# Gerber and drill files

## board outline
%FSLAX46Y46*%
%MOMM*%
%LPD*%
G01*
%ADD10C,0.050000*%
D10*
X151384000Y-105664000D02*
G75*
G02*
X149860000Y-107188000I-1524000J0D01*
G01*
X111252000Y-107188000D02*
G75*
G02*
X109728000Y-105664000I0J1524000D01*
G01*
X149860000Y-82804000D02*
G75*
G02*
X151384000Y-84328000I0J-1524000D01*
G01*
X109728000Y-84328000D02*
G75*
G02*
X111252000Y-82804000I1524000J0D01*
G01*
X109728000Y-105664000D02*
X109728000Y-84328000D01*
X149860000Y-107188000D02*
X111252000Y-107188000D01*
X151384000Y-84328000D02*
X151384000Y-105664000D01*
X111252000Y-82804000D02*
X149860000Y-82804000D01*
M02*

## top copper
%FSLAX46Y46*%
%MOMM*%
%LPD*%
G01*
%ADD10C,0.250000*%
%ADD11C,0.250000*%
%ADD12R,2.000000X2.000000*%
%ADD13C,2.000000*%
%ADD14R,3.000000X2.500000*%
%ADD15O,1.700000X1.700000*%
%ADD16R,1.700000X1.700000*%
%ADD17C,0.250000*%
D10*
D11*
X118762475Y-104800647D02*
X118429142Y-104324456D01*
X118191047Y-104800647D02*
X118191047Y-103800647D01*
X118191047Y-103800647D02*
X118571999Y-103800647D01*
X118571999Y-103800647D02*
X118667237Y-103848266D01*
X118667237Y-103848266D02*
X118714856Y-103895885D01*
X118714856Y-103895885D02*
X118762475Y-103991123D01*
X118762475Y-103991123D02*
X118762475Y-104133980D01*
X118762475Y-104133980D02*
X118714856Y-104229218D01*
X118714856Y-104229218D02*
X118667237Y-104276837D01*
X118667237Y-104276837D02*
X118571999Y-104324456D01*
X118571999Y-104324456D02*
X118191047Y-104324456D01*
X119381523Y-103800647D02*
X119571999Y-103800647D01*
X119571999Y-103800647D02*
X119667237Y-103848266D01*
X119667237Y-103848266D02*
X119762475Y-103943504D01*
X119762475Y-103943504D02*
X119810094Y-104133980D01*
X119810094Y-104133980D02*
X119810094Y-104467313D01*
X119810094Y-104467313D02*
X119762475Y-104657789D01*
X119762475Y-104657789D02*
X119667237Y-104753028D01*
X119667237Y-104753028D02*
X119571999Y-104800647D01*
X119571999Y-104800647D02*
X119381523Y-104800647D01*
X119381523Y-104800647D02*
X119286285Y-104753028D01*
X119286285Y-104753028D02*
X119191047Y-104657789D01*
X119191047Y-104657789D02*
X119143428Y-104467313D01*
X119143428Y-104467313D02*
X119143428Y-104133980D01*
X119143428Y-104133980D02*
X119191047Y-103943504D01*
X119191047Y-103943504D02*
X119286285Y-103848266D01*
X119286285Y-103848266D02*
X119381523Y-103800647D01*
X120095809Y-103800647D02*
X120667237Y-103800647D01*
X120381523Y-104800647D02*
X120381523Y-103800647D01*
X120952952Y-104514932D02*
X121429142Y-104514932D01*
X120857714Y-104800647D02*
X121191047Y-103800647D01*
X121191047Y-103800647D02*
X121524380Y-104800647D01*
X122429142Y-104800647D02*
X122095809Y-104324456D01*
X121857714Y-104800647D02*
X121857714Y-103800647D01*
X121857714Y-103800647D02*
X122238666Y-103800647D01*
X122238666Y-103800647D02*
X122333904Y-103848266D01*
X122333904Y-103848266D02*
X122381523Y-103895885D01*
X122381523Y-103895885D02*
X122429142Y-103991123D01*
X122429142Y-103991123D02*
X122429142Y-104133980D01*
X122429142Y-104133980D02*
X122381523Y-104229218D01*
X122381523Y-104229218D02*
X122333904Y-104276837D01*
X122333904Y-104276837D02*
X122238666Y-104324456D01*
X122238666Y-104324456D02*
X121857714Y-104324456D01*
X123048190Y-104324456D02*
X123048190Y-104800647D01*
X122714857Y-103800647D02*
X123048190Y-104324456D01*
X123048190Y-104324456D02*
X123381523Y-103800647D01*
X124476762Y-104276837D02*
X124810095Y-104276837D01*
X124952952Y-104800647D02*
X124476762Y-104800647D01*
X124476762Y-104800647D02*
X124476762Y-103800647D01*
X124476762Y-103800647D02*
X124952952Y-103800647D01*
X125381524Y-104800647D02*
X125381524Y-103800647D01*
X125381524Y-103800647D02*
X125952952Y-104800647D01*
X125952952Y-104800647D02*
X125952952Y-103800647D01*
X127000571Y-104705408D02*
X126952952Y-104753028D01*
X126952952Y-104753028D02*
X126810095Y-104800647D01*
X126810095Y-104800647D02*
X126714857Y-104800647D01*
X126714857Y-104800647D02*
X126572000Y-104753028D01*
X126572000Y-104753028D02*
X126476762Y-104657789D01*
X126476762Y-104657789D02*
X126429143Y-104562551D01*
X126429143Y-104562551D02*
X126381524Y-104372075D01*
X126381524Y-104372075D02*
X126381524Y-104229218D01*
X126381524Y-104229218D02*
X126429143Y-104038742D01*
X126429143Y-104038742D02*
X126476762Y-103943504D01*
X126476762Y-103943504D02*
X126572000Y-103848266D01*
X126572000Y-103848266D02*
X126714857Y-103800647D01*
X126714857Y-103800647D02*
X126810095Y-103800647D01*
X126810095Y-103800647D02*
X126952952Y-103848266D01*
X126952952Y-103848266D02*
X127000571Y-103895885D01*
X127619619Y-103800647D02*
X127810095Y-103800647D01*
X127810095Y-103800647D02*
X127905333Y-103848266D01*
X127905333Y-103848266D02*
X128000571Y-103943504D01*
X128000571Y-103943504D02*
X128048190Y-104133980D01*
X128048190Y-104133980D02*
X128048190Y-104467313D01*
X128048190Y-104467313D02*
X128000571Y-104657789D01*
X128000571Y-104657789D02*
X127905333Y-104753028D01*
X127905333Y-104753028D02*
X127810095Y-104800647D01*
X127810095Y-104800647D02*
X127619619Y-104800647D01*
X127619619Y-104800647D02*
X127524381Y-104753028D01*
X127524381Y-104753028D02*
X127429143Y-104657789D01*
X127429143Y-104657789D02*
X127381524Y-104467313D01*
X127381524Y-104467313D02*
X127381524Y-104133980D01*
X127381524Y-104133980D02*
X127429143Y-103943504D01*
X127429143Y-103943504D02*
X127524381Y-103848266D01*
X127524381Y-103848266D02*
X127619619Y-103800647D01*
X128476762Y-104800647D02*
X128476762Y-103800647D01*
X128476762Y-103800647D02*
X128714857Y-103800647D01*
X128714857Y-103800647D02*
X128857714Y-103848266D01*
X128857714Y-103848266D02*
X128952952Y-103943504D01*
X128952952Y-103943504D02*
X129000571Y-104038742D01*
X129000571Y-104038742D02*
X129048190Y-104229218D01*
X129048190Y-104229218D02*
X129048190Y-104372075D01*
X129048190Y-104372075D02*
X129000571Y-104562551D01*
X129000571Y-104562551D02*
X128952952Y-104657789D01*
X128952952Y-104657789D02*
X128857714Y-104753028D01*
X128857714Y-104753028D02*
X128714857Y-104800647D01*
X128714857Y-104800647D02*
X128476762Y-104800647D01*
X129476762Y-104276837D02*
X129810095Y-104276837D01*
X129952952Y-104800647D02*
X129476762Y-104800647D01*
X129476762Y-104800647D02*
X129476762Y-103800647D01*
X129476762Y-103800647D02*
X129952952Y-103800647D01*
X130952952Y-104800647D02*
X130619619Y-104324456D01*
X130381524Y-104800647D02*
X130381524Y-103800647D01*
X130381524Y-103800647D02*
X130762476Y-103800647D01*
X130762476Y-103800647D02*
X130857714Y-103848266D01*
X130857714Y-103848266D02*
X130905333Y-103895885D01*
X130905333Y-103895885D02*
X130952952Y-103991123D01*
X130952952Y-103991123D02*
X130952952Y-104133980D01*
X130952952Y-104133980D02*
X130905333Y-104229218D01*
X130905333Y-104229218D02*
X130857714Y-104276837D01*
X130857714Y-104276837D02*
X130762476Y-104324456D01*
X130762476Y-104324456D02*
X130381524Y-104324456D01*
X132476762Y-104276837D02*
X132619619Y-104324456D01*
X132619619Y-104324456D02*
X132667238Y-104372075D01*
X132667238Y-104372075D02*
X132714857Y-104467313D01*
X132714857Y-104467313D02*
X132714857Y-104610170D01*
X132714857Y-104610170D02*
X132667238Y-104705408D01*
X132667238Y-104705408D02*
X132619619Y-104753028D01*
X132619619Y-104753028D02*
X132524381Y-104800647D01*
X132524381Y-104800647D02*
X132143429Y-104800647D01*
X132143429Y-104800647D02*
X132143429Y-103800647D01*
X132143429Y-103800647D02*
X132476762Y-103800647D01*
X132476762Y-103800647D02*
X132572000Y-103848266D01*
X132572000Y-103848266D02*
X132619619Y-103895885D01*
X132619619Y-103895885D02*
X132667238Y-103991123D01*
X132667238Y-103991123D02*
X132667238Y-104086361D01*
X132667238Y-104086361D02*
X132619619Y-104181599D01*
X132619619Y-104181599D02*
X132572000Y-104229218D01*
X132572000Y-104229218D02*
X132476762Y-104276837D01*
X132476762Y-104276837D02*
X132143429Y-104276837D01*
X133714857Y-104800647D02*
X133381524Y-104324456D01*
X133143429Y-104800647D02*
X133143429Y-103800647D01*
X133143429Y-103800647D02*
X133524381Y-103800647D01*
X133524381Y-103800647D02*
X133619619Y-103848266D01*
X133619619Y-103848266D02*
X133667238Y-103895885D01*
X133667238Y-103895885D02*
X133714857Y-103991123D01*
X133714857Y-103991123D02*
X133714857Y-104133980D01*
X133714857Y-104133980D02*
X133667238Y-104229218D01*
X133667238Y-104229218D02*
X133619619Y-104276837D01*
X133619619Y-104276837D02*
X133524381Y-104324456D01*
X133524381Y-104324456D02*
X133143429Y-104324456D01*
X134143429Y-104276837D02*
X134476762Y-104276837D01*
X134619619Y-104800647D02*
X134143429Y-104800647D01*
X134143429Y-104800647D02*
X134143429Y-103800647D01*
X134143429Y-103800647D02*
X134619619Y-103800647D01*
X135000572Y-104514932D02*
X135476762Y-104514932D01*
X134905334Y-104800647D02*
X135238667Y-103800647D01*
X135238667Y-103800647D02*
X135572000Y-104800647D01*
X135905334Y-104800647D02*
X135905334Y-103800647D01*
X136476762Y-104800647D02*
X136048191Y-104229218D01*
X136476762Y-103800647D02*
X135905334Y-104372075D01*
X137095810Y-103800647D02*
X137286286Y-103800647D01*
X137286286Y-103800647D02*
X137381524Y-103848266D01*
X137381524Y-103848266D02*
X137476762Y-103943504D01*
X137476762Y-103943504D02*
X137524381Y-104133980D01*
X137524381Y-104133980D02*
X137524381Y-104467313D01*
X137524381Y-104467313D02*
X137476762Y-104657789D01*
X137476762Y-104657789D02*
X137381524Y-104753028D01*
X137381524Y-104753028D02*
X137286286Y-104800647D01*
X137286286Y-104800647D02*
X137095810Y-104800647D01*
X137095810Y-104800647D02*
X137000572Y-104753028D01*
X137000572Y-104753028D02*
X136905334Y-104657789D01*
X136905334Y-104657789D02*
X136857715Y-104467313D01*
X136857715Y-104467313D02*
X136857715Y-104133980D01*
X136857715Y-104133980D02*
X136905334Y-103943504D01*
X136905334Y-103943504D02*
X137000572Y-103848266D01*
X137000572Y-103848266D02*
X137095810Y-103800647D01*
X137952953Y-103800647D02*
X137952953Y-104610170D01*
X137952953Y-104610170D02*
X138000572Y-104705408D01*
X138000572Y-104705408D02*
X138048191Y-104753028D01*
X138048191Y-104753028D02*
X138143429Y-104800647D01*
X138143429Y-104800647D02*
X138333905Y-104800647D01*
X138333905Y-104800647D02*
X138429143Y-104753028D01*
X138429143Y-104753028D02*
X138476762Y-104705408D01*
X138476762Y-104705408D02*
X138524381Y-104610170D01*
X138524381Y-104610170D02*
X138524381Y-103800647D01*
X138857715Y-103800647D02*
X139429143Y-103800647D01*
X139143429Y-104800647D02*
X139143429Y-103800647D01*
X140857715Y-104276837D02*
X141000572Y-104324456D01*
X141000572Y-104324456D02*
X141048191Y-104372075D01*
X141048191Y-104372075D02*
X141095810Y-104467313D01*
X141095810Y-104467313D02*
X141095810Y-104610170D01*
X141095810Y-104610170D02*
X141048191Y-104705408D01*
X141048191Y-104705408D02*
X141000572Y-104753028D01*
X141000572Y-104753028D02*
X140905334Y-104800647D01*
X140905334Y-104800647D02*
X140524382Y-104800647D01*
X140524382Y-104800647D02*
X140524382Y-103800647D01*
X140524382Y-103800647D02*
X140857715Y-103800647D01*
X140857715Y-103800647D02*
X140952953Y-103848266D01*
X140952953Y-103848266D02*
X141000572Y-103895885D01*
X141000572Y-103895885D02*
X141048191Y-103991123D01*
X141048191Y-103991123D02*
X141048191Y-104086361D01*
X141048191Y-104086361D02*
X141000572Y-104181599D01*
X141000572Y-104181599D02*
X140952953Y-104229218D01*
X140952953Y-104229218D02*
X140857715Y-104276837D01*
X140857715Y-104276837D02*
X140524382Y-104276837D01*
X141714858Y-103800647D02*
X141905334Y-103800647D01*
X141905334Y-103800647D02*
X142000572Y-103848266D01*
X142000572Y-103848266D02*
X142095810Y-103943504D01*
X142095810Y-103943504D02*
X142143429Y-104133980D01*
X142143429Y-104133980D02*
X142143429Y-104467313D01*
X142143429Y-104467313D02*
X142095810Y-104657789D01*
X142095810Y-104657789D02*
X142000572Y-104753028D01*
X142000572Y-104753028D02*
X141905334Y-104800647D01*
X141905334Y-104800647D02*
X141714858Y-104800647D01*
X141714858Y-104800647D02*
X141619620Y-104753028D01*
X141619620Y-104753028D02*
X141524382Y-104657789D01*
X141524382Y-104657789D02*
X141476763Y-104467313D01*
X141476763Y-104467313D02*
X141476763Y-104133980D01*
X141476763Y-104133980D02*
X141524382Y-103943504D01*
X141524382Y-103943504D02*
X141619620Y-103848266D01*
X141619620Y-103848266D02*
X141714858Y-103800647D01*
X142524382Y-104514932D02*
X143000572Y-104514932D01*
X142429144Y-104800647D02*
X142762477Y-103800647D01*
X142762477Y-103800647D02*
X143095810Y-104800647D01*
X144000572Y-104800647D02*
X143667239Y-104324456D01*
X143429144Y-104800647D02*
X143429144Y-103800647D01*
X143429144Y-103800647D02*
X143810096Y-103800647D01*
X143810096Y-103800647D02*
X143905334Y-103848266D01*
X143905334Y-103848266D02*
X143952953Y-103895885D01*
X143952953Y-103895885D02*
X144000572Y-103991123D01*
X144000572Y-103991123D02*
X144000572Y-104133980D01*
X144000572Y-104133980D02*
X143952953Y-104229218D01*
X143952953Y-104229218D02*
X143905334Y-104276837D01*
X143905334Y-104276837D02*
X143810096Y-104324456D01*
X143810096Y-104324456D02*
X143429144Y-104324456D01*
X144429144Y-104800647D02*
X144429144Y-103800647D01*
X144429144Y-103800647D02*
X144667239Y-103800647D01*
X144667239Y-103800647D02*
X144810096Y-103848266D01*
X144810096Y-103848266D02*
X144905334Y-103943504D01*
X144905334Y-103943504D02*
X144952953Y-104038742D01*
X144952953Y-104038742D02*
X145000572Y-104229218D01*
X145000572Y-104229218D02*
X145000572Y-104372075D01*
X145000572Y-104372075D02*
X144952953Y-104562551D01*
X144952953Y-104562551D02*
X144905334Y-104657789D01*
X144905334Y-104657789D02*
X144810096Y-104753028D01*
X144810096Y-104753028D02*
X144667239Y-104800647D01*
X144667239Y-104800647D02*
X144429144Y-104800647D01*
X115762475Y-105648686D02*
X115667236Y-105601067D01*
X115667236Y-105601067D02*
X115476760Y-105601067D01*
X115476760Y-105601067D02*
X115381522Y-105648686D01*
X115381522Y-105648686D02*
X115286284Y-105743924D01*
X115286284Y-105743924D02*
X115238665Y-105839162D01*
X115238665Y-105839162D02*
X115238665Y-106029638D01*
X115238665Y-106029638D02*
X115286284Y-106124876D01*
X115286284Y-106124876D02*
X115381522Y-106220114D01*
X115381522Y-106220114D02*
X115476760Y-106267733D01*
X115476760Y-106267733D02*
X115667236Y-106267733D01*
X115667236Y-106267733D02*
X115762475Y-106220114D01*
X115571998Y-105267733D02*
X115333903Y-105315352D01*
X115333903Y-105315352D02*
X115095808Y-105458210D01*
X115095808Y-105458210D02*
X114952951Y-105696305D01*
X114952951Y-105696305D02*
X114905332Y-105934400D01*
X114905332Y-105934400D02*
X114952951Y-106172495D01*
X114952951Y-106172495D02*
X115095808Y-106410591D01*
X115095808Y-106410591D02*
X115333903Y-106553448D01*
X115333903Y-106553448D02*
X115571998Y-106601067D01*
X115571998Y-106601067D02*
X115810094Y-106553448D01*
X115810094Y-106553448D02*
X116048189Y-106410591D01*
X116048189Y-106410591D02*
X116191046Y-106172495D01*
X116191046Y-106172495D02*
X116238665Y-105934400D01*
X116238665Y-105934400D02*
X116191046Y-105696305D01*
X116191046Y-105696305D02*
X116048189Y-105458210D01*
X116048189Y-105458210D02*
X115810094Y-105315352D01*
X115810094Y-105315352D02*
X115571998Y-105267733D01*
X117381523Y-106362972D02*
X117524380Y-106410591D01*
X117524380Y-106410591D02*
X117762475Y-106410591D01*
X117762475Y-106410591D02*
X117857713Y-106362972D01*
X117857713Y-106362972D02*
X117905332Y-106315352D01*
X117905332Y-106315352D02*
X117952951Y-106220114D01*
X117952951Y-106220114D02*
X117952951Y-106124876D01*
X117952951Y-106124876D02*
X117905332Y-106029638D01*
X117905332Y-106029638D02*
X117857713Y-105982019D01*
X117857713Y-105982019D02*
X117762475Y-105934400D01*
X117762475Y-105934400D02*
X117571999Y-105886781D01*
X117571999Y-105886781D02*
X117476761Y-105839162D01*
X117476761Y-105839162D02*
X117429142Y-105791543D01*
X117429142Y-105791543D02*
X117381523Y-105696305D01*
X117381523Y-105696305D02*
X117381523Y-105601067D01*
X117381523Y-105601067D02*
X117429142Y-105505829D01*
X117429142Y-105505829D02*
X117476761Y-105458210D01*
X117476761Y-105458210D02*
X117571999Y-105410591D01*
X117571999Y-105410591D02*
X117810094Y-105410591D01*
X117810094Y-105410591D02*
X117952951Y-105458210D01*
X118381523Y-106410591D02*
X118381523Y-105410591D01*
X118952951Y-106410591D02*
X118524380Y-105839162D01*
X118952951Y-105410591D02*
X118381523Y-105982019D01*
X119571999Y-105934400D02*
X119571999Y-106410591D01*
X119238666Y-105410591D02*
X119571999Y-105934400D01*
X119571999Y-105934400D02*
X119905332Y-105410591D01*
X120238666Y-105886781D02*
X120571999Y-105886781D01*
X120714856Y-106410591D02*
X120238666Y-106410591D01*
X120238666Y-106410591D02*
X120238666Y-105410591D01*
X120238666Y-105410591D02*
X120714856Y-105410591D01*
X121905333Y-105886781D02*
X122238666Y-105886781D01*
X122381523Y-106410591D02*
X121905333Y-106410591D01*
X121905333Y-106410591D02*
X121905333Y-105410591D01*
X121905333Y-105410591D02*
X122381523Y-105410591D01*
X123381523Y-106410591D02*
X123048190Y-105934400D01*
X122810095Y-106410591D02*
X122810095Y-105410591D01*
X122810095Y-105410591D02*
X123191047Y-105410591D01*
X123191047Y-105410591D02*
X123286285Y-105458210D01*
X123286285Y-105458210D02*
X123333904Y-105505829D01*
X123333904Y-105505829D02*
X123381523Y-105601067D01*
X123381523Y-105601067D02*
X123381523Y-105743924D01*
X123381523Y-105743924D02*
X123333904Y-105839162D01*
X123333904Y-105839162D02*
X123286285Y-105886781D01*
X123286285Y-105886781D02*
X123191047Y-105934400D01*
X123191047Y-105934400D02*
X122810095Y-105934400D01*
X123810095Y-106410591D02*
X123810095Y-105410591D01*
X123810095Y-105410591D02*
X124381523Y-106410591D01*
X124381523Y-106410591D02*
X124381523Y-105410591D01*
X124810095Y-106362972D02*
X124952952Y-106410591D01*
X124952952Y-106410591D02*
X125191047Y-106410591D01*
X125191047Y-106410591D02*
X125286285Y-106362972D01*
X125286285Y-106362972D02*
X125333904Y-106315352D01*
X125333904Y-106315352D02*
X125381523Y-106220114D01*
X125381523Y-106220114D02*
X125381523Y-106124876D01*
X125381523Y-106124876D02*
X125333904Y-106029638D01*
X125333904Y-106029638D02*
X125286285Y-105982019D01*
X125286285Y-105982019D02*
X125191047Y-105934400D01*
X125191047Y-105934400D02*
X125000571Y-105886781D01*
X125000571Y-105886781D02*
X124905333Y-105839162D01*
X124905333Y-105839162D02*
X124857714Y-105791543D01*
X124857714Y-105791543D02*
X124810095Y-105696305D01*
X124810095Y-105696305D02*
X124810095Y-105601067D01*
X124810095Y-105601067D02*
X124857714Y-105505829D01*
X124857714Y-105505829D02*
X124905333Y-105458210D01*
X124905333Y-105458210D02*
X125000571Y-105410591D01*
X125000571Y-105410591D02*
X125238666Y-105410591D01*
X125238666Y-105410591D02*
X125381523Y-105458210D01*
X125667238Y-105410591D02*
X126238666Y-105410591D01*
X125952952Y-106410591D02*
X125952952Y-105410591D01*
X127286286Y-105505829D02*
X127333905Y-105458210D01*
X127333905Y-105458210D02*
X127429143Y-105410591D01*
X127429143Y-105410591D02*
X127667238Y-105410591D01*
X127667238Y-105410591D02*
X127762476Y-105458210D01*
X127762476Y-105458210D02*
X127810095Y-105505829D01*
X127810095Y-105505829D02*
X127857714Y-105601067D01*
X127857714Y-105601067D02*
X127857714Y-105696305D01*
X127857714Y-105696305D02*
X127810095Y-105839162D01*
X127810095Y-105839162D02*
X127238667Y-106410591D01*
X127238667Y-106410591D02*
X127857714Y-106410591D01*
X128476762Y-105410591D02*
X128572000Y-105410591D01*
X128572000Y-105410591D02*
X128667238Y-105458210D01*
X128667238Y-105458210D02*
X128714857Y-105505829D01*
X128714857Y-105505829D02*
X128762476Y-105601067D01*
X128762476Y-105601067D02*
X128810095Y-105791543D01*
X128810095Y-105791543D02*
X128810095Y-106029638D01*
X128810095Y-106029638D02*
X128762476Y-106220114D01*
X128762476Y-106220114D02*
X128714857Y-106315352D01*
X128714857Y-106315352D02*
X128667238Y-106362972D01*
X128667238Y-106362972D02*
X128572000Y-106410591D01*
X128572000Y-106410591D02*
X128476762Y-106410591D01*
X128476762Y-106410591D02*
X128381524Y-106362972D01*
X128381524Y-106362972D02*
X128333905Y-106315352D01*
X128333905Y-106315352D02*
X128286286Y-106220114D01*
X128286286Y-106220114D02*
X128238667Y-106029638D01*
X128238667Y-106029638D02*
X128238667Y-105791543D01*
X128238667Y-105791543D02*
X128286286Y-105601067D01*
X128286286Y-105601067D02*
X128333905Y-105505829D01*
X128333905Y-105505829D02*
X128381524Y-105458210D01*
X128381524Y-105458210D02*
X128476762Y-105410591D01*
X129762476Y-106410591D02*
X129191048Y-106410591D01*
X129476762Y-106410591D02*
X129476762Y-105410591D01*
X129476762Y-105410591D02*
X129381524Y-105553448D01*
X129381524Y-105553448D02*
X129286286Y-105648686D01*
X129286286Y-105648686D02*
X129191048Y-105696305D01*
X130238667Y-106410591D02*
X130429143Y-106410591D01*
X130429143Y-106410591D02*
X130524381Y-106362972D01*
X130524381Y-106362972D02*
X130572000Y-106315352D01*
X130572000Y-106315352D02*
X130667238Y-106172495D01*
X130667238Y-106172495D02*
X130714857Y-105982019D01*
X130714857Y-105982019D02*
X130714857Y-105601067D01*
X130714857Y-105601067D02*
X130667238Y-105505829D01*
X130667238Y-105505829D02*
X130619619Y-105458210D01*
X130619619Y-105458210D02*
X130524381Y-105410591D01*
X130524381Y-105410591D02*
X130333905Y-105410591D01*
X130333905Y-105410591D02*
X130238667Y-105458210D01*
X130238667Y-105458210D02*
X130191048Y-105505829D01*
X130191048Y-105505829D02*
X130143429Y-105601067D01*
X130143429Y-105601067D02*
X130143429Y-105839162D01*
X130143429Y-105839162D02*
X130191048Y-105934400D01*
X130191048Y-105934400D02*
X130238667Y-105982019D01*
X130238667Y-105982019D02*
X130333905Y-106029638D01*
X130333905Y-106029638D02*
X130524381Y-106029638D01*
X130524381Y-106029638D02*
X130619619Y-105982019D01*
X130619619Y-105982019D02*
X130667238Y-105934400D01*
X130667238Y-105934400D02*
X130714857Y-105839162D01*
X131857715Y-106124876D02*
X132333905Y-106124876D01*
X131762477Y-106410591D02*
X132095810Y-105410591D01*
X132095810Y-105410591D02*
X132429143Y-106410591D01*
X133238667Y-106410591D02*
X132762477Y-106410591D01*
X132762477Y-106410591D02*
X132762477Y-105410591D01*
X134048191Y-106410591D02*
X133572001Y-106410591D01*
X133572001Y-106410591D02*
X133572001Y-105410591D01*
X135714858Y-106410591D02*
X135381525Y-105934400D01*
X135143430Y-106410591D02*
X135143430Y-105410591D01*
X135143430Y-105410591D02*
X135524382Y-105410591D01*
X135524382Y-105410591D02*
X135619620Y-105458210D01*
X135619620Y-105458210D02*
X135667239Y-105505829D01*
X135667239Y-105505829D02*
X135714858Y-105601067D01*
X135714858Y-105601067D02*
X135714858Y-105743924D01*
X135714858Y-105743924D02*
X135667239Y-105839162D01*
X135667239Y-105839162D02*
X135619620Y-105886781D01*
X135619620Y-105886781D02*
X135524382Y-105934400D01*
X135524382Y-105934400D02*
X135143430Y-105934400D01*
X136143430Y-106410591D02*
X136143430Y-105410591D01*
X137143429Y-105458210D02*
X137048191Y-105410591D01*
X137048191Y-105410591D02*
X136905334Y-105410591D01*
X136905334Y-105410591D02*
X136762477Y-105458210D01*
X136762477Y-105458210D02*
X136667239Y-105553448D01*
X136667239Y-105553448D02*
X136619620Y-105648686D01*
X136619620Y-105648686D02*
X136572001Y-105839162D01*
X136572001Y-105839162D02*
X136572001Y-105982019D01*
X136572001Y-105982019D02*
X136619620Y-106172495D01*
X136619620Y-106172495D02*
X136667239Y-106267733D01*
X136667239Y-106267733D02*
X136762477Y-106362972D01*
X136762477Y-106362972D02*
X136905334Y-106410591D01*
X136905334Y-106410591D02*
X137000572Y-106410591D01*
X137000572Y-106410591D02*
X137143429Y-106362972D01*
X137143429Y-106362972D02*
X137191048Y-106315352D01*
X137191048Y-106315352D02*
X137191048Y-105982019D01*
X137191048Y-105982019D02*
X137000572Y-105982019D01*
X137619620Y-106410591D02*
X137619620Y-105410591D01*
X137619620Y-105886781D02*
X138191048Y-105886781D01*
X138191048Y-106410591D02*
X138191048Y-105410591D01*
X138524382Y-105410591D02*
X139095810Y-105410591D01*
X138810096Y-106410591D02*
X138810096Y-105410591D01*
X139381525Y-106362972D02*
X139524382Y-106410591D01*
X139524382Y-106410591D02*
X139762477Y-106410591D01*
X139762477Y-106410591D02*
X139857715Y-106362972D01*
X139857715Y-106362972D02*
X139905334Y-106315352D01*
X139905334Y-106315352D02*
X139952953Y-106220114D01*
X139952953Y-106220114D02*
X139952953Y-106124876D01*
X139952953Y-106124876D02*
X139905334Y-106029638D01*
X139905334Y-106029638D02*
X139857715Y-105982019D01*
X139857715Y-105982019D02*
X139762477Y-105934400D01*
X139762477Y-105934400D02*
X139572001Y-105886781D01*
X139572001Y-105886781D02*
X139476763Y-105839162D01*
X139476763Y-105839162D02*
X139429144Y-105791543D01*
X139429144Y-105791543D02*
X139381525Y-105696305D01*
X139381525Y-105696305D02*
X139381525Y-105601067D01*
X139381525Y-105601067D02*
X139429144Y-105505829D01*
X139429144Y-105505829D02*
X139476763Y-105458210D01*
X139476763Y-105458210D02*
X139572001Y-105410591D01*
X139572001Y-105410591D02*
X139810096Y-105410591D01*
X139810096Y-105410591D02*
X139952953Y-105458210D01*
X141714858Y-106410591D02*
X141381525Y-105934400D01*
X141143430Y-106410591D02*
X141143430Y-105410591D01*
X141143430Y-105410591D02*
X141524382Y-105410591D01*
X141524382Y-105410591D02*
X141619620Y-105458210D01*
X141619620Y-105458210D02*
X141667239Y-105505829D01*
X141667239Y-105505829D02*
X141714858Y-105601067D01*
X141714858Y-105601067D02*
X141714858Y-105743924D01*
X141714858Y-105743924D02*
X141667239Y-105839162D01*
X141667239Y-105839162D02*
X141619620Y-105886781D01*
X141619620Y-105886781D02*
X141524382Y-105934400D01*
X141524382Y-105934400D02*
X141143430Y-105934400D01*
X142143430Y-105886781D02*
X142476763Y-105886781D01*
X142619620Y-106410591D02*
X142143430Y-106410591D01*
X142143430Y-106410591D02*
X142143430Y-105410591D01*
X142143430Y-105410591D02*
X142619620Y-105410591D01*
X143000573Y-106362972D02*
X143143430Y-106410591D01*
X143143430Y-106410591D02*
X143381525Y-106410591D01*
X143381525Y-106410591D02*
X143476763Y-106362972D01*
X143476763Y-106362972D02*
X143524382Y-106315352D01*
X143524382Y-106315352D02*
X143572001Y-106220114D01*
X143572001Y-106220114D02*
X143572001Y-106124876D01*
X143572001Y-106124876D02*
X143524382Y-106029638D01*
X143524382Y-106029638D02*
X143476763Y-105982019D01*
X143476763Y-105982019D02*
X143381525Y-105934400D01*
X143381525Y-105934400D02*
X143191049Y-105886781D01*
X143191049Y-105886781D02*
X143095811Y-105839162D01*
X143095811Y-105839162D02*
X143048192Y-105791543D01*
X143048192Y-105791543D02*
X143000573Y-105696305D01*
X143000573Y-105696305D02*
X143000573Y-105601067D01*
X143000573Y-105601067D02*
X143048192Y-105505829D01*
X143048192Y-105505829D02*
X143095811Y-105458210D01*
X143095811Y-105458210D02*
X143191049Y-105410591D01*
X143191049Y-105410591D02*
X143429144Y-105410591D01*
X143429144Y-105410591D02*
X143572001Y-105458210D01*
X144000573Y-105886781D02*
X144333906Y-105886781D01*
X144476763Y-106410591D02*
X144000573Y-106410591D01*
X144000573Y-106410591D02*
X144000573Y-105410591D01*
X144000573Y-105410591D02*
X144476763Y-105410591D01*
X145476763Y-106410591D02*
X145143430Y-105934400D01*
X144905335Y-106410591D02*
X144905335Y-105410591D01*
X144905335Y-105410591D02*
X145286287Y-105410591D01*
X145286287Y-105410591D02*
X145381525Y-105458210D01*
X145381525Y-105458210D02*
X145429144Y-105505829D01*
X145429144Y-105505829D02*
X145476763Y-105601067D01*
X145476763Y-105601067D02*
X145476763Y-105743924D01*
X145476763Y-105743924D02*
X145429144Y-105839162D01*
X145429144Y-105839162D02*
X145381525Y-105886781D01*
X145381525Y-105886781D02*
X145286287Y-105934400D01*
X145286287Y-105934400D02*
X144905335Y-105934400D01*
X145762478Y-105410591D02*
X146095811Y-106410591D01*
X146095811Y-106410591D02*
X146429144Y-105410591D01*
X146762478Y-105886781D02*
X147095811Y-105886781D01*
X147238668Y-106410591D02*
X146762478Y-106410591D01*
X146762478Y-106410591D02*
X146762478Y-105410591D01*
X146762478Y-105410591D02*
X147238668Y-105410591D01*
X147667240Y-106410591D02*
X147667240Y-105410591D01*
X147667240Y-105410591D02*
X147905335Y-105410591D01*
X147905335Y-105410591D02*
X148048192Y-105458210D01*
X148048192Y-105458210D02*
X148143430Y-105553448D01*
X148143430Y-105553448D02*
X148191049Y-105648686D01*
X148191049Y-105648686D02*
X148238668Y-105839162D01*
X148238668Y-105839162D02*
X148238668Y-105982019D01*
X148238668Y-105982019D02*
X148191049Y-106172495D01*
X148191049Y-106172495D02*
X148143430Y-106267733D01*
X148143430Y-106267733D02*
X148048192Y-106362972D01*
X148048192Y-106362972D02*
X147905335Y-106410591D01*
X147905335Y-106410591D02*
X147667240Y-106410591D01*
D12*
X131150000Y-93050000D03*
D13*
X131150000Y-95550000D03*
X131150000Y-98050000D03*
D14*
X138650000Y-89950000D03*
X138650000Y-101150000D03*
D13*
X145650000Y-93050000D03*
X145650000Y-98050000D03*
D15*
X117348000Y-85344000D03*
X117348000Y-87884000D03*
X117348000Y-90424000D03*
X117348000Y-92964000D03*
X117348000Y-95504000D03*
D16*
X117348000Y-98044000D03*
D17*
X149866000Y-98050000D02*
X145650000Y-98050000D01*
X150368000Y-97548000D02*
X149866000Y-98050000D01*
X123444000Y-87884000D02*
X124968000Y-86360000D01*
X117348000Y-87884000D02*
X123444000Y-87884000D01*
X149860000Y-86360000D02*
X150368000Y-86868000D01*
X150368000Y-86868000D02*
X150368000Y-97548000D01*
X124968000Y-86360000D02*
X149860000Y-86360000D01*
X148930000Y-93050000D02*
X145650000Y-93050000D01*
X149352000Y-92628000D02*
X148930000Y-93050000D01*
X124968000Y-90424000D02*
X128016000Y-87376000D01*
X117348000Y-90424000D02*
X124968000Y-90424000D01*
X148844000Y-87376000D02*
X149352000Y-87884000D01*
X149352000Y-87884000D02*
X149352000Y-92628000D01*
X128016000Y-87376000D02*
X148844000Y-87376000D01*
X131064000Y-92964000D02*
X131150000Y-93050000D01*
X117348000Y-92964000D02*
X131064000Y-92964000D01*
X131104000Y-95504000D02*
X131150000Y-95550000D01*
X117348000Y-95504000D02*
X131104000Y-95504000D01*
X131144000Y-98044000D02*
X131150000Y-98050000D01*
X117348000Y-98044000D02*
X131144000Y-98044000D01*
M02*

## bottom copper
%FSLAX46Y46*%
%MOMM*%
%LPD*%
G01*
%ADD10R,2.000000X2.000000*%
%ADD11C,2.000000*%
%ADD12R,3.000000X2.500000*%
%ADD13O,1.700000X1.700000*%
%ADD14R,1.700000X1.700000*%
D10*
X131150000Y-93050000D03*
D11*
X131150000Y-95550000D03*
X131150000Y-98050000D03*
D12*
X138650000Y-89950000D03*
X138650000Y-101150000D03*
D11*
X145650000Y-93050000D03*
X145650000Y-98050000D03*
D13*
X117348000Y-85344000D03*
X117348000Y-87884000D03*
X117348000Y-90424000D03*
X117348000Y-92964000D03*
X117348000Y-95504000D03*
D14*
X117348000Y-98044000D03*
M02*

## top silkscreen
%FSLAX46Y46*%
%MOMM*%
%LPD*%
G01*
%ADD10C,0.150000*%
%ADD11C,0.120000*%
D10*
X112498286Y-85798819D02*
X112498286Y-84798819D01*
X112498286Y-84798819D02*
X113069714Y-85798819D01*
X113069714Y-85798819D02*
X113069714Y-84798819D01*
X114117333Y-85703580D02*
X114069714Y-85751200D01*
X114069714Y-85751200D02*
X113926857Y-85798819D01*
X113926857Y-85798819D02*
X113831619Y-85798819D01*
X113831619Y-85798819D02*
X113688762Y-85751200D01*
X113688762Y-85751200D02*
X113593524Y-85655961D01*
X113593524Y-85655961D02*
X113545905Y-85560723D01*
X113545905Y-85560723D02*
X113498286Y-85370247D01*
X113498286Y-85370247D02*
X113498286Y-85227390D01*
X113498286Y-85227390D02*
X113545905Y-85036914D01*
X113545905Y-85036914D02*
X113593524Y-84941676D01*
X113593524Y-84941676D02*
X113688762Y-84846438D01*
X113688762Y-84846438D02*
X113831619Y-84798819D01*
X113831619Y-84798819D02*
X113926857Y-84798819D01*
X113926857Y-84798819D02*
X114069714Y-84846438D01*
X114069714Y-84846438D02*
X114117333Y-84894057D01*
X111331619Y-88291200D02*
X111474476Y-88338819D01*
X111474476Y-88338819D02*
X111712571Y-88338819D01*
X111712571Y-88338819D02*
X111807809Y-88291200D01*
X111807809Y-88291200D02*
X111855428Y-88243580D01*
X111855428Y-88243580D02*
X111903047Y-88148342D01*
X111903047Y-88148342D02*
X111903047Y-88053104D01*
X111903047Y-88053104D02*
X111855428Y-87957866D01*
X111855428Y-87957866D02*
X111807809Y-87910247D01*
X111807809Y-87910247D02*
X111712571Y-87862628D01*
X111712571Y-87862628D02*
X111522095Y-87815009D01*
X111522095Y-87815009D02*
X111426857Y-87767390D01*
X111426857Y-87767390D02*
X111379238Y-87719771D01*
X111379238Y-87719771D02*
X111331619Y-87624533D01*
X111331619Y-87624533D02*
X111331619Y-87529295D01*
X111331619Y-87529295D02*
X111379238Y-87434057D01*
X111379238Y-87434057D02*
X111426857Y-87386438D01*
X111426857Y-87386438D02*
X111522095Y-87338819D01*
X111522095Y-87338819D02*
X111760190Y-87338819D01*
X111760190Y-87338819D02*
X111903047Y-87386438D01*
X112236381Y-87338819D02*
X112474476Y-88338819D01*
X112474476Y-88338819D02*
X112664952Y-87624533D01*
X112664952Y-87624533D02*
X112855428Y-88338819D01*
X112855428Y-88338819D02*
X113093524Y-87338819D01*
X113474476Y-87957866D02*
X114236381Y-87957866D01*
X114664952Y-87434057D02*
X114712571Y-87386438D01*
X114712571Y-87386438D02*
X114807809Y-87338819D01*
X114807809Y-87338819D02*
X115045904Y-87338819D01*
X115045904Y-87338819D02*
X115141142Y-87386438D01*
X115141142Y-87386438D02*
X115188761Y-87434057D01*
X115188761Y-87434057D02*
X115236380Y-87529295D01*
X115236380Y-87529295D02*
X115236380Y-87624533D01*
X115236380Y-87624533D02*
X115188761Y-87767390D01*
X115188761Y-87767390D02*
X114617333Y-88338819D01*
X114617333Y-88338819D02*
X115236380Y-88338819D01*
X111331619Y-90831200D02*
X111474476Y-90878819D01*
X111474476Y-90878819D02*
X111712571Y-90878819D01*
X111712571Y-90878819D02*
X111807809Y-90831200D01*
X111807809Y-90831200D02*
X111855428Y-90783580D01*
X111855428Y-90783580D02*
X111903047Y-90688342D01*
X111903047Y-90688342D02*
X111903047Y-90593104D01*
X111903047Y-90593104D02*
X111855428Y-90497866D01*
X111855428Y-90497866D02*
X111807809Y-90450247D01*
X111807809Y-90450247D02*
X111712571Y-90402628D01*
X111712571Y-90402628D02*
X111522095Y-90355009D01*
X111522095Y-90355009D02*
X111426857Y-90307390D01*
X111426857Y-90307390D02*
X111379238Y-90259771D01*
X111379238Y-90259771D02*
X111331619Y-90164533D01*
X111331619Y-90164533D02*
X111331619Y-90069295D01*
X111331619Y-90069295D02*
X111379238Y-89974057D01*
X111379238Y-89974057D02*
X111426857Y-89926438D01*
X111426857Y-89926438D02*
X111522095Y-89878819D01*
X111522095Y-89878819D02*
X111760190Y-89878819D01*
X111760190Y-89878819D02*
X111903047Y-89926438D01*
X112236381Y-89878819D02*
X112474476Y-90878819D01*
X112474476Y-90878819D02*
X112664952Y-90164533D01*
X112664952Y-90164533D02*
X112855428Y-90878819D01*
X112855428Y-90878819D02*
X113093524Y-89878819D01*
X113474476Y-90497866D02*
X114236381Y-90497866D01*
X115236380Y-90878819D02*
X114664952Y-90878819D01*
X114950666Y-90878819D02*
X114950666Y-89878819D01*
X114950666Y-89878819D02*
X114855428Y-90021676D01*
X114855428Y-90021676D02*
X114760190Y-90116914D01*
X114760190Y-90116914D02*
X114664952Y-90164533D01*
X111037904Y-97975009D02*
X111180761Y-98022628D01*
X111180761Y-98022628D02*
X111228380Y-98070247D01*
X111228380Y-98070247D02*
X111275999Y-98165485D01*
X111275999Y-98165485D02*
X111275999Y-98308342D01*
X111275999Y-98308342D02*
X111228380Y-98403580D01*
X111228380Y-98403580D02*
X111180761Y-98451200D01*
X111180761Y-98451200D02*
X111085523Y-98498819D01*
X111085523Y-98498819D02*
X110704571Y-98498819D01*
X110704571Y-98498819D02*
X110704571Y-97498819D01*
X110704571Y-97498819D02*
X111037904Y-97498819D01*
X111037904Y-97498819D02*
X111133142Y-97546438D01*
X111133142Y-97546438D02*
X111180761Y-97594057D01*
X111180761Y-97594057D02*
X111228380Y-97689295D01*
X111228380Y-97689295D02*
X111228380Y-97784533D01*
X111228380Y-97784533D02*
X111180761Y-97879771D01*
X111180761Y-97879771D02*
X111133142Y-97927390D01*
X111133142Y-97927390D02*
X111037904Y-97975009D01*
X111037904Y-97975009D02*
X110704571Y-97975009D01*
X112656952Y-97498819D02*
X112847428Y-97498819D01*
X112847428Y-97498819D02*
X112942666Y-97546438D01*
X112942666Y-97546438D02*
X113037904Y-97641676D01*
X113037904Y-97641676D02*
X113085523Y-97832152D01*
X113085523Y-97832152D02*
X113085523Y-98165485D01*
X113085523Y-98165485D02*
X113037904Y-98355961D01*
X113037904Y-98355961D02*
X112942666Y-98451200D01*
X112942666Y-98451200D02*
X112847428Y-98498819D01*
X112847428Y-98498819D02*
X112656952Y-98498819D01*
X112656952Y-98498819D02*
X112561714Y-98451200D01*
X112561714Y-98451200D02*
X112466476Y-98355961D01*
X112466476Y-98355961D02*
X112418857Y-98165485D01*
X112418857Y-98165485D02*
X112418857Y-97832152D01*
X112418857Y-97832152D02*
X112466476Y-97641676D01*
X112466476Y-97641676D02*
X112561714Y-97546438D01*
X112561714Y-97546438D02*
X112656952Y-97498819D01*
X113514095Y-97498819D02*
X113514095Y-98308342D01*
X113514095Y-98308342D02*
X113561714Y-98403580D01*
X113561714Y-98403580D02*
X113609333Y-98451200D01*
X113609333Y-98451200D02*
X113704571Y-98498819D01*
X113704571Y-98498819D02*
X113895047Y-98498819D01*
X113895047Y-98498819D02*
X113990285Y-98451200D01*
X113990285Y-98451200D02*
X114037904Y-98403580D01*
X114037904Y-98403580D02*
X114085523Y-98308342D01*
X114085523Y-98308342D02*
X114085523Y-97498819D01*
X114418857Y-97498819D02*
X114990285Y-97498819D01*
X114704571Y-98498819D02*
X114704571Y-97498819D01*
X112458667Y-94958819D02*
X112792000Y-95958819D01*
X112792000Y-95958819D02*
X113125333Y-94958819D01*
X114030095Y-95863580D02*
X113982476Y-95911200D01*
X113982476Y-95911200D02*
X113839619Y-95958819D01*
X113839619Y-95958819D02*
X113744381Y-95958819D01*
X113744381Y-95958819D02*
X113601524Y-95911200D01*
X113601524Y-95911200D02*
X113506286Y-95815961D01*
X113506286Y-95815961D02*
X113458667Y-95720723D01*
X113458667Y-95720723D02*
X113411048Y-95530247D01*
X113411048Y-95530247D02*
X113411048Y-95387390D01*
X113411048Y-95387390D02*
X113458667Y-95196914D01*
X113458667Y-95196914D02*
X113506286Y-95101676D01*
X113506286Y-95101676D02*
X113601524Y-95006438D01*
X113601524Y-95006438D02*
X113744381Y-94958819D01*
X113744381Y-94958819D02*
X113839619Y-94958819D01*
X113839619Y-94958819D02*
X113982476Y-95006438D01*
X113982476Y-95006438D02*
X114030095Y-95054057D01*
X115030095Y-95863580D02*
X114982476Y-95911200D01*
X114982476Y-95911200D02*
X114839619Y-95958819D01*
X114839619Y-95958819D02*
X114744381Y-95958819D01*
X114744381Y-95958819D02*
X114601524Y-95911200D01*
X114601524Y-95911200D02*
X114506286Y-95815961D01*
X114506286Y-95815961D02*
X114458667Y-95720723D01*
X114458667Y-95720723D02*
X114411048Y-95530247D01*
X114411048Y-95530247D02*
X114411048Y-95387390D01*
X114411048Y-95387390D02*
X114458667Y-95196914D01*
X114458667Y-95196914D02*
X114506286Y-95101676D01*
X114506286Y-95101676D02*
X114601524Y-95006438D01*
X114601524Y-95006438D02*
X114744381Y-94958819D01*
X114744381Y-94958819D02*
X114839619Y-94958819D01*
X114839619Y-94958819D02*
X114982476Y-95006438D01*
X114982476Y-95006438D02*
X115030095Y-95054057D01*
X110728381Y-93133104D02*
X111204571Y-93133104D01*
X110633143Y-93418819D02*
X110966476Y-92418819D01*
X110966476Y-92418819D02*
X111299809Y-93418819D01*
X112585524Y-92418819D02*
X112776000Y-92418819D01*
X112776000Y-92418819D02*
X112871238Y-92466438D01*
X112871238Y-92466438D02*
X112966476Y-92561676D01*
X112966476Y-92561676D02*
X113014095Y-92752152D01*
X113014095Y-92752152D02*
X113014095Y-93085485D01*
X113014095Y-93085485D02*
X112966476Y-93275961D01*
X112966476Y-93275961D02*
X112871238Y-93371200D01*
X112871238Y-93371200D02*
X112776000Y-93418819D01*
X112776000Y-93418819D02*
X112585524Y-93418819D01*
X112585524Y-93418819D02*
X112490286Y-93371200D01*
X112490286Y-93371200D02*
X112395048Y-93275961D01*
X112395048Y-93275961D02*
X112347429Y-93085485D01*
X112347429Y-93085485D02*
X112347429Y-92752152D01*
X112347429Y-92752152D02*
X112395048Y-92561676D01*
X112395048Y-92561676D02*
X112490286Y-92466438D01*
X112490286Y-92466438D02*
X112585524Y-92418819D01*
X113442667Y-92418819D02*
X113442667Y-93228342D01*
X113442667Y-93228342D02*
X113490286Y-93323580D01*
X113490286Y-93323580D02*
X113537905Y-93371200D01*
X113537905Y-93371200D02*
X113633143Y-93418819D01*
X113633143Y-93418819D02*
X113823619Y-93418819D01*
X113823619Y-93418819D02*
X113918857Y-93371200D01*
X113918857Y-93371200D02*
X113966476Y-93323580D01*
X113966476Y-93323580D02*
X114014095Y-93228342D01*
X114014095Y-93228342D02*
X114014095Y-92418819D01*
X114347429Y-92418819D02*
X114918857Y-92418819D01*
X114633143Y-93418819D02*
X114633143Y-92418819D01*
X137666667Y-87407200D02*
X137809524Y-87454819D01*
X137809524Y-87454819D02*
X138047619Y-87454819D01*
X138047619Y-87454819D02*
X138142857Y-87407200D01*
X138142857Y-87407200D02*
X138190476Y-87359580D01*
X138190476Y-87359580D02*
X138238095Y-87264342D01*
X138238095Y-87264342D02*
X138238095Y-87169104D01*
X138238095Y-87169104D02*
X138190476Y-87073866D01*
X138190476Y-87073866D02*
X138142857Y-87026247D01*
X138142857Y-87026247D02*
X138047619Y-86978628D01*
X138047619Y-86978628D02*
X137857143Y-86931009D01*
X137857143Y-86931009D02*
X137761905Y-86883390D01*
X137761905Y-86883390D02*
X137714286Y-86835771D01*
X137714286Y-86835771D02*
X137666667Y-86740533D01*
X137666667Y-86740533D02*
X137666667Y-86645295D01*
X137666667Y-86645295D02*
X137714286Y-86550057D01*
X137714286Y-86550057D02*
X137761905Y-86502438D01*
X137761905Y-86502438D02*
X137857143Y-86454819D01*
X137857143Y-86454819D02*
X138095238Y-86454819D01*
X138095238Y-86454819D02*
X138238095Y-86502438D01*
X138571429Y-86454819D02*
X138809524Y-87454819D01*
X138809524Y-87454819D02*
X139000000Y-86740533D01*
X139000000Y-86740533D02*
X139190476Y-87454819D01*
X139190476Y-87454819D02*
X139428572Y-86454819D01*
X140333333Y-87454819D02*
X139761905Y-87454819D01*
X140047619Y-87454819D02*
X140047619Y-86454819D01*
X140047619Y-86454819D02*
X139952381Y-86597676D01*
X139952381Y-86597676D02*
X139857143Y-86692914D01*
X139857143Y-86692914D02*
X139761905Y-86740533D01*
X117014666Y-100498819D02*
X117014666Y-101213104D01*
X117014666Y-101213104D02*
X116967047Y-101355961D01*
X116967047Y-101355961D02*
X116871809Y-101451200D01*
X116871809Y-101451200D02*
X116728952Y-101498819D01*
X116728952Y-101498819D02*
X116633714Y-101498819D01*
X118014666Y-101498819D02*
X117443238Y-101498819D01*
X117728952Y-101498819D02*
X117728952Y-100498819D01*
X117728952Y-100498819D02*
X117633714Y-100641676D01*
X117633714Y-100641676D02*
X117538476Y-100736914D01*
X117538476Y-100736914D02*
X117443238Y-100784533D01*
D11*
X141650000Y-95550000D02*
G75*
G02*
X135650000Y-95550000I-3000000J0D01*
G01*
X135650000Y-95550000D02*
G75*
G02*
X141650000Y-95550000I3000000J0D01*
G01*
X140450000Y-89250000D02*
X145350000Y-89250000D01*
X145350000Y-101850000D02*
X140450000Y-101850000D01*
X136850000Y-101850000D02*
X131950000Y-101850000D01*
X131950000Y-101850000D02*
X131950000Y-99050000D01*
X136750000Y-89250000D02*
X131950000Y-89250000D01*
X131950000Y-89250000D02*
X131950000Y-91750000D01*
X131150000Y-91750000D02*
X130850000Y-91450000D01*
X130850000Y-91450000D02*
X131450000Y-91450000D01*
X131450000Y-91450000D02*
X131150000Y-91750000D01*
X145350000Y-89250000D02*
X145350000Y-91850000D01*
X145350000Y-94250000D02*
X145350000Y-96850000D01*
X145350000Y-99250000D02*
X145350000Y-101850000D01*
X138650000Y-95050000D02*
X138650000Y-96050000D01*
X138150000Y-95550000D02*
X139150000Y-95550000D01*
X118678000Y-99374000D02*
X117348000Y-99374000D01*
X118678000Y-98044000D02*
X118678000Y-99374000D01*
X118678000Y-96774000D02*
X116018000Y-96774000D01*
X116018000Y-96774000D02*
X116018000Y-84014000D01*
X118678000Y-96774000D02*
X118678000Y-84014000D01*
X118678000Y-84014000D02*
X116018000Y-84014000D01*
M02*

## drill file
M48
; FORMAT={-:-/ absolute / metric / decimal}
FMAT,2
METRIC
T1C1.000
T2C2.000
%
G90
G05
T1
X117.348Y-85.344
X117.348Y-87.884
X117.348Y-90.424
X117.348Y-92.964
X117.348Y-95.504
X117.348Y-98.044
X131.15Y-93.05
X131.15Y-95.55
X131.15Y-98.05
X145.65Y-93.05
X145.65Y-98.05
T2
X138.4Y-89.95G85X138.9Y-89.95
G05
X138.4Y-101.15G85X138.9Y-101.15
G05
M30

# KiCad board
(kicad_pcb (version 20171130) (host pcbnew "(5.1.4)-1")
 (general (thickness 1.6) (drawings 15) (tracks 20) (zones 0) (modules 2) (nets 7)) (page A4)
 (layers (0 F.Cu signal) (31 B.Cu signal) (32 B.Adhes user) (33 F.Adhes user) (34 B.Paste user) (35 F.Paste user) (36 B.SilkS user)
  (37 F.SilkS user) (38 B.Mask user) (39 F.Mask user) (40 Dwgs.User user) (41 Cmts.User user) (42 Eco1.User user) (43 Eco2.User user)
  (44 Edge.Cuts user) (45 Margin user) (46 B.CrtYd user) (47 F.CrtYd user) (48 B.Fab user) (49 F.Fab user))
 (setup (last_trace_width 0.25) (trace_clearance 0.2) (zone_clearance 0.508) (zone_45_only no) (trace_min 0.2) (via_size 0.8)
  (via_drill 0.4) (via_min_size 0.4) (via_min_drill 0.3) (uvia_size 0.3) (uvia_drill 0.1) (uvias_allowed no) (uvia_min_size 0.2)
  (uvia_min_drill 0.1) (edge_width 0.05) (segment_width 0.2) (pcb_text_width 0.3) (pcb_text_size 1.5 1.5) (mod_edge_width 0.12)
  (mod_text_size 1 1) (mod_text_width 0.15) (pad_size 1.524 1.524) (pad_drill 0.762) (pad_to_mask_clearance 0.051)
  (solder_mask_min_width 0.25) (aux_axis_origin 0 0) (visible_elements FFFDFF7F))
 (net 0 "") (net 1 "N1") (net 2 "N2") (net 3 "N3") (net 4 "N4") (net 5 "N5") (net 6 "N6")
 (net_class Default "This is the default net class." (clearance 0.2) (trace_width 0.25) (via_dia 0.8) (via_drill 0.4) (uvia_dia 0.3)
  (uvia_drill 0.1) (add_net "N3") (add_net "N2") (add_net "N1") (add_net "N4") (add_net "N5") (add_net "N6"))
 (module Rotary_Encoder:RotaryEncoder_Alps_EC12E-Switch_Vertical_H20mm (layer F.Cu) (at 131.15 93.05)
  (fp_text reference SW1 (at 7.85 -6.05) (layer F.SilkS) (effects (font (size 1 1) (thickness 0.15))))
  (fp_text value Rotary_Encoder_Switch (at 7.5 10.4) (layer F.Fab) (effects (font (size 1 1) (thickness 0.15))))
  (fp_circle (center 7.5 2.5) (end 10.5 2.5) (layer F.SilkS) (width 0.12))
  (fp_line (start 9.3 -3.8) (end 14.2 -3.8) (layer F.SilkS) (width 0.12))
  (fp_line (start 14.2 8.8) (end 9.3 8.8) (layer F.SilkS) (width 0.12))
  (fp_line (start 5.7 8.8) (end 0.8 8.8) (layer F.SilkS) (width 0.12))
  (fp_line (start 0.8 8.8) (end 0.8 6) (layer F.SilkS) (width 0.12))
  (fp_line (start 5.6 -3.8) (end 0.8 -3.8) (layer F.SilkS) (width 0.12))
  (fp_line (start 0.8 -3.8) (end 0.8 -1.3) (layer F.SilkS) (width 0.12))
  (fp_line (start 0 -1.3) (end -0.3 -1.6) (layer F.SilkS) (width 0.12))
  (fp_line (start -0.3 -1.6) (end 0.3 -1.6) (layer F.SilkS) (width 0.12))
  (fp_line (start 0.3 -1.6) (end 0 -1.3) (layer F.SilkS) (width 0.12))
  (fp_line (start 14.2 -3.8) (end 14.2 -1.2) (layer F.SilkS) (width 0.12))
  (fp_line (start 14.2 1.2) (end 14.2 3.8) (layer F.SilkS) (width 0.12))
  (fp_line (start 14.2 6.2) (end 14.2 8.8) (layer F.SilkS) (width 0.12))
  (fp_line (start 7.5 2) (end 7.5 3) (layer F.SilkS) (width 0.12))
  (fp_line (start 7 2.5) (end 8 2.5) (layer F.SilkS) (width 0.12))
  (pad A thru_hole rect (at 0 0) (size 2 2) (drill 1) (layers *.Cu *.Mask) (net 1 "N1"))
  (pad C thru_hole circle (at 0 2.5) (size 2 2) (drill 1) (layers *.Cu *.Mask) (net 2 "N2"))
  (pad B thru_hole circle (at 0 5) (size 2 2) (drill 1) (layers *.Cu *.Mask) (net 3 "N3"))
  (pad MP thru_hole rect (at 7.5 -3.1) (size 3 2.5) (drill oval 2.5 2) (layers *.Cu *.Mask))
  (pad MP thru_hole rect (at 7.5 8.1) (size 3 2.5) (drill oval 2.5 2) (layers *.Cu *.Mask))
  (pad S1 thru_hole circle (at 14.5 0) (size 2 2) (drill 1) (layers *.Cu *.Mask) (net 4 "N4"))
  (pad S2 thru_hole circle (at 14.5 5) (size 2 2) (drill 1) (layers *.Cu *.Mask) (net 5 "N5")))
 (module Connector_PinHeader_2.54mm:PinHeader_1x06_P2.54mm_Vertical (layer F.Cu) (at 117.348 98.044 180)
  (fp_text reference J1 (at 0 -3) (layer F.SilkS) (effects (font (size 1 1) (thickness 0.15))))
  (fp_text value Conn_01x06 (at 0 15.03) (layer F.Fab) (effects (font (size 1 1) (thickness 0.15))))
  (fp_line (start -1.33 -1.33) (end 0 -1.33) (layer F.SilkS) (width 0.12))
  (fp_line (start -1.33 0) (end -1.33 -1.33) (layer F.SilkS) (width 0.12))
  (fp_line (start -1.33 1.27) (end 1.33 1.27) (layer F.SilkS) (width 0.12))
  (fp_line (start 1.33 1.27) (end 1.33 14.03) (layer F.SilkS) (width 0.12))
  (fp_line (start -1.33 1.27) (end -1.33 14.03) (layer F.SilkS) (width 0.12))
  (fp_line (start -1.33 14.03) (end 1.33 14.03) (layer F.SilkS) (width 0.12))
  (pad 6 thru_hole oval (at 0 12.7 180) (size 1.7 1.7) (drill 1) (layers *.Cu *.Mask) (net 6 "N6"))
  (pad 5 thru_hole oval (at 0 10.16 180) (size 1.7 1.7) (drill 1) (layers *.Cu *.Mask) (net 5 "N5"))
  (pad 4 thru_hole oval (at 0 7.62 180) (size 1.7 1.7) (drill 1) (layers *.Cu *.Mask) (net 4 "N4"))
  (pad 3 thru_hole oval (at 0 5.08 180) (size 1.7 1.7) (drill 1) (layers *.Cu *.Mask) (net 1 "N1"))
  (pad 2 thru_hole oval (at 0 2.54 180) (size 1.7 1.7) (drill 1) (layers *.Cu *.Mask) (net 2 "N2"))
  (pad 1 thru_hole rect (at 0 0 180) (size 1.7 1.7) (drill 1) (layers *.Cu *.Mask) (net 3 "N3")))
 (gr_arc (start 149.86 105.664) (end 149.86 107.188) (angle -90) (layer Edge.Cuts) (width 0.05))
 (gr_arc (start 111.252 105.664) (end 109.728 105.664) (angle -90) (layer Edge.Cuts) (width 0.05))
 (gr_arc (start 149.86 84.328) (end 151.384 84.328) (angle -90) (layer Edge.Cuts) (width 0.05))
 (gr_arc (start 111.252 84.328) (end 111.252 82.804) (angle -90) (layer Edge.Cuts) (width 0.05))
 (gr_line (start 109.728 105.664) (end 109.728 84.328) (layer Edge.Cuts) (width 0.05))
 (gr_line (start 149.86 107.188) (end 111.252 107.188) (layer Edge.Cuts) (width 0.05))
 (gr_line (start 151.384 84.328) (end 151.384 105.664) (layer Edge.Cuts) (width 0.05))
 (gr_line (start 111.252 82.804) (end 149.86 82.804) (layer Edge.Cuts) (width 0.05))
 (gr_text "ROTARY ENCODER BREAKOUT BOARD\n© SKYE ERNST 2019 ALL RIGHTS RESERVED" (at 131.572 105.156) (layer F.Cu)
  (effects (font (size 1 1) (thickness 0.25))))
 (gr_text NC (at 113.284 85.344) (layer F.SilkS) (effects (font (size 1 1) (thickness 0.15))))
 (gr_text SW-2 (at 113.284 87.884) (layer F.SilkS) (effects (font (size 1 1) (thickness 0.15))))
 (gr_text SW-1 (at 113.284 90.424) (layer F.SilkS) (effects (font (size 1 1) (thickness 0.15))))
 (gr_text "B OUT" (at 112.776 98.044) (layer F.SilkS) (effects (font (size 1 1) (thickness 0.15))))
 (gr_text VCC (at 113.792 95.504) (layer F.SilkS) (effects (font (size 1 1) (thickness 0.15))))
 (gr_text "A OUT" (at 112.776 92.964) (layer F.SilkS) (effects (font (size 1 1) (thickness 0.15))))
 (segment (start 149.866 98.05) (end 145.65 98.05) (width 0.25) (layer F.Cu) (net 5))
 (segment (start 150.368 97.548) (end 149.866 98.05) (width 0.25) (layer F.Cu) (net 5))
 (segment (start 123.444 87.884) (end 124.968 86.36) (width 0.25) (layer F.Cu) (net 5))
 (segment (start 117.348 87.884) (end 123.444 87.884) (width 0.25) (layer F.Cu) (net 5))
 (segment (start 149.86 86.36) (end 150.368 86.868) (width 0.25) (layer F.Cu) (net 5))
 (segment (start 150.368 86.868) (end 150.368 97.548) (width 0.25) (layer F.Cu) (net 5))
 (segment (start 124.968 86.36) (end 149.86 86.36) (width 0.25) (layer F.Cu) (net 5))
 (segment (start 148.93 93.05) (end 145.65 93.05) (width 0.25) (layer F.Cu) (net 4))
 (segment (start 149.352 92.628) (end 148.93 93.05) (width 0.25) (layer F.Cu) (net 4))
 (segment (start 124.968 90.424) (end 128.016 87.376) (width 0.25) (layer F.Cu) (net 4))
 (segment (start 117.348 90.424) (end 124.968 90.424) (width 0.25) (layer F.Cu) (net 4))
 (segment (start 148.844 87.376) (end 149.352 87.884) (width 0.25) (layer F.Cu) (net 4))
 (segment (start 149.352 87.884) (end 149.352 92.628) (width 0.25) (layer F.Cu) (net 4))
 (segment (start 128.016 87.376) (end 148.844 87.376) (width 0.25) (layer F.Cu) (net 4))
 (segment (start 131.064 92.964) (end 131.15 93.05) (width 0.25) (layer F.Cu) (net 1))
 (segment (start 117.348 92.964) (end 131.064 92.964) (width 0.25) (layer F.Cu) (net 1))
 (segment (start 131.104 95.504) (end 131.15 95.55) (width 0.25) (layer F.Cu) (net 2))
 (segment (start 117.348 95.504) (end 131.104 95.504) (width 0.25) (layer F.Cu) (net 2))
 (segment (start 131.144 98.044) (end 131.15 98.05) (width 0.25) (layer F.Cu) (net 3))
 (segment (start 117.348 98.044) (end 131.144 98.044) (width 0.25) (layer F.Cu) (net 3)))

